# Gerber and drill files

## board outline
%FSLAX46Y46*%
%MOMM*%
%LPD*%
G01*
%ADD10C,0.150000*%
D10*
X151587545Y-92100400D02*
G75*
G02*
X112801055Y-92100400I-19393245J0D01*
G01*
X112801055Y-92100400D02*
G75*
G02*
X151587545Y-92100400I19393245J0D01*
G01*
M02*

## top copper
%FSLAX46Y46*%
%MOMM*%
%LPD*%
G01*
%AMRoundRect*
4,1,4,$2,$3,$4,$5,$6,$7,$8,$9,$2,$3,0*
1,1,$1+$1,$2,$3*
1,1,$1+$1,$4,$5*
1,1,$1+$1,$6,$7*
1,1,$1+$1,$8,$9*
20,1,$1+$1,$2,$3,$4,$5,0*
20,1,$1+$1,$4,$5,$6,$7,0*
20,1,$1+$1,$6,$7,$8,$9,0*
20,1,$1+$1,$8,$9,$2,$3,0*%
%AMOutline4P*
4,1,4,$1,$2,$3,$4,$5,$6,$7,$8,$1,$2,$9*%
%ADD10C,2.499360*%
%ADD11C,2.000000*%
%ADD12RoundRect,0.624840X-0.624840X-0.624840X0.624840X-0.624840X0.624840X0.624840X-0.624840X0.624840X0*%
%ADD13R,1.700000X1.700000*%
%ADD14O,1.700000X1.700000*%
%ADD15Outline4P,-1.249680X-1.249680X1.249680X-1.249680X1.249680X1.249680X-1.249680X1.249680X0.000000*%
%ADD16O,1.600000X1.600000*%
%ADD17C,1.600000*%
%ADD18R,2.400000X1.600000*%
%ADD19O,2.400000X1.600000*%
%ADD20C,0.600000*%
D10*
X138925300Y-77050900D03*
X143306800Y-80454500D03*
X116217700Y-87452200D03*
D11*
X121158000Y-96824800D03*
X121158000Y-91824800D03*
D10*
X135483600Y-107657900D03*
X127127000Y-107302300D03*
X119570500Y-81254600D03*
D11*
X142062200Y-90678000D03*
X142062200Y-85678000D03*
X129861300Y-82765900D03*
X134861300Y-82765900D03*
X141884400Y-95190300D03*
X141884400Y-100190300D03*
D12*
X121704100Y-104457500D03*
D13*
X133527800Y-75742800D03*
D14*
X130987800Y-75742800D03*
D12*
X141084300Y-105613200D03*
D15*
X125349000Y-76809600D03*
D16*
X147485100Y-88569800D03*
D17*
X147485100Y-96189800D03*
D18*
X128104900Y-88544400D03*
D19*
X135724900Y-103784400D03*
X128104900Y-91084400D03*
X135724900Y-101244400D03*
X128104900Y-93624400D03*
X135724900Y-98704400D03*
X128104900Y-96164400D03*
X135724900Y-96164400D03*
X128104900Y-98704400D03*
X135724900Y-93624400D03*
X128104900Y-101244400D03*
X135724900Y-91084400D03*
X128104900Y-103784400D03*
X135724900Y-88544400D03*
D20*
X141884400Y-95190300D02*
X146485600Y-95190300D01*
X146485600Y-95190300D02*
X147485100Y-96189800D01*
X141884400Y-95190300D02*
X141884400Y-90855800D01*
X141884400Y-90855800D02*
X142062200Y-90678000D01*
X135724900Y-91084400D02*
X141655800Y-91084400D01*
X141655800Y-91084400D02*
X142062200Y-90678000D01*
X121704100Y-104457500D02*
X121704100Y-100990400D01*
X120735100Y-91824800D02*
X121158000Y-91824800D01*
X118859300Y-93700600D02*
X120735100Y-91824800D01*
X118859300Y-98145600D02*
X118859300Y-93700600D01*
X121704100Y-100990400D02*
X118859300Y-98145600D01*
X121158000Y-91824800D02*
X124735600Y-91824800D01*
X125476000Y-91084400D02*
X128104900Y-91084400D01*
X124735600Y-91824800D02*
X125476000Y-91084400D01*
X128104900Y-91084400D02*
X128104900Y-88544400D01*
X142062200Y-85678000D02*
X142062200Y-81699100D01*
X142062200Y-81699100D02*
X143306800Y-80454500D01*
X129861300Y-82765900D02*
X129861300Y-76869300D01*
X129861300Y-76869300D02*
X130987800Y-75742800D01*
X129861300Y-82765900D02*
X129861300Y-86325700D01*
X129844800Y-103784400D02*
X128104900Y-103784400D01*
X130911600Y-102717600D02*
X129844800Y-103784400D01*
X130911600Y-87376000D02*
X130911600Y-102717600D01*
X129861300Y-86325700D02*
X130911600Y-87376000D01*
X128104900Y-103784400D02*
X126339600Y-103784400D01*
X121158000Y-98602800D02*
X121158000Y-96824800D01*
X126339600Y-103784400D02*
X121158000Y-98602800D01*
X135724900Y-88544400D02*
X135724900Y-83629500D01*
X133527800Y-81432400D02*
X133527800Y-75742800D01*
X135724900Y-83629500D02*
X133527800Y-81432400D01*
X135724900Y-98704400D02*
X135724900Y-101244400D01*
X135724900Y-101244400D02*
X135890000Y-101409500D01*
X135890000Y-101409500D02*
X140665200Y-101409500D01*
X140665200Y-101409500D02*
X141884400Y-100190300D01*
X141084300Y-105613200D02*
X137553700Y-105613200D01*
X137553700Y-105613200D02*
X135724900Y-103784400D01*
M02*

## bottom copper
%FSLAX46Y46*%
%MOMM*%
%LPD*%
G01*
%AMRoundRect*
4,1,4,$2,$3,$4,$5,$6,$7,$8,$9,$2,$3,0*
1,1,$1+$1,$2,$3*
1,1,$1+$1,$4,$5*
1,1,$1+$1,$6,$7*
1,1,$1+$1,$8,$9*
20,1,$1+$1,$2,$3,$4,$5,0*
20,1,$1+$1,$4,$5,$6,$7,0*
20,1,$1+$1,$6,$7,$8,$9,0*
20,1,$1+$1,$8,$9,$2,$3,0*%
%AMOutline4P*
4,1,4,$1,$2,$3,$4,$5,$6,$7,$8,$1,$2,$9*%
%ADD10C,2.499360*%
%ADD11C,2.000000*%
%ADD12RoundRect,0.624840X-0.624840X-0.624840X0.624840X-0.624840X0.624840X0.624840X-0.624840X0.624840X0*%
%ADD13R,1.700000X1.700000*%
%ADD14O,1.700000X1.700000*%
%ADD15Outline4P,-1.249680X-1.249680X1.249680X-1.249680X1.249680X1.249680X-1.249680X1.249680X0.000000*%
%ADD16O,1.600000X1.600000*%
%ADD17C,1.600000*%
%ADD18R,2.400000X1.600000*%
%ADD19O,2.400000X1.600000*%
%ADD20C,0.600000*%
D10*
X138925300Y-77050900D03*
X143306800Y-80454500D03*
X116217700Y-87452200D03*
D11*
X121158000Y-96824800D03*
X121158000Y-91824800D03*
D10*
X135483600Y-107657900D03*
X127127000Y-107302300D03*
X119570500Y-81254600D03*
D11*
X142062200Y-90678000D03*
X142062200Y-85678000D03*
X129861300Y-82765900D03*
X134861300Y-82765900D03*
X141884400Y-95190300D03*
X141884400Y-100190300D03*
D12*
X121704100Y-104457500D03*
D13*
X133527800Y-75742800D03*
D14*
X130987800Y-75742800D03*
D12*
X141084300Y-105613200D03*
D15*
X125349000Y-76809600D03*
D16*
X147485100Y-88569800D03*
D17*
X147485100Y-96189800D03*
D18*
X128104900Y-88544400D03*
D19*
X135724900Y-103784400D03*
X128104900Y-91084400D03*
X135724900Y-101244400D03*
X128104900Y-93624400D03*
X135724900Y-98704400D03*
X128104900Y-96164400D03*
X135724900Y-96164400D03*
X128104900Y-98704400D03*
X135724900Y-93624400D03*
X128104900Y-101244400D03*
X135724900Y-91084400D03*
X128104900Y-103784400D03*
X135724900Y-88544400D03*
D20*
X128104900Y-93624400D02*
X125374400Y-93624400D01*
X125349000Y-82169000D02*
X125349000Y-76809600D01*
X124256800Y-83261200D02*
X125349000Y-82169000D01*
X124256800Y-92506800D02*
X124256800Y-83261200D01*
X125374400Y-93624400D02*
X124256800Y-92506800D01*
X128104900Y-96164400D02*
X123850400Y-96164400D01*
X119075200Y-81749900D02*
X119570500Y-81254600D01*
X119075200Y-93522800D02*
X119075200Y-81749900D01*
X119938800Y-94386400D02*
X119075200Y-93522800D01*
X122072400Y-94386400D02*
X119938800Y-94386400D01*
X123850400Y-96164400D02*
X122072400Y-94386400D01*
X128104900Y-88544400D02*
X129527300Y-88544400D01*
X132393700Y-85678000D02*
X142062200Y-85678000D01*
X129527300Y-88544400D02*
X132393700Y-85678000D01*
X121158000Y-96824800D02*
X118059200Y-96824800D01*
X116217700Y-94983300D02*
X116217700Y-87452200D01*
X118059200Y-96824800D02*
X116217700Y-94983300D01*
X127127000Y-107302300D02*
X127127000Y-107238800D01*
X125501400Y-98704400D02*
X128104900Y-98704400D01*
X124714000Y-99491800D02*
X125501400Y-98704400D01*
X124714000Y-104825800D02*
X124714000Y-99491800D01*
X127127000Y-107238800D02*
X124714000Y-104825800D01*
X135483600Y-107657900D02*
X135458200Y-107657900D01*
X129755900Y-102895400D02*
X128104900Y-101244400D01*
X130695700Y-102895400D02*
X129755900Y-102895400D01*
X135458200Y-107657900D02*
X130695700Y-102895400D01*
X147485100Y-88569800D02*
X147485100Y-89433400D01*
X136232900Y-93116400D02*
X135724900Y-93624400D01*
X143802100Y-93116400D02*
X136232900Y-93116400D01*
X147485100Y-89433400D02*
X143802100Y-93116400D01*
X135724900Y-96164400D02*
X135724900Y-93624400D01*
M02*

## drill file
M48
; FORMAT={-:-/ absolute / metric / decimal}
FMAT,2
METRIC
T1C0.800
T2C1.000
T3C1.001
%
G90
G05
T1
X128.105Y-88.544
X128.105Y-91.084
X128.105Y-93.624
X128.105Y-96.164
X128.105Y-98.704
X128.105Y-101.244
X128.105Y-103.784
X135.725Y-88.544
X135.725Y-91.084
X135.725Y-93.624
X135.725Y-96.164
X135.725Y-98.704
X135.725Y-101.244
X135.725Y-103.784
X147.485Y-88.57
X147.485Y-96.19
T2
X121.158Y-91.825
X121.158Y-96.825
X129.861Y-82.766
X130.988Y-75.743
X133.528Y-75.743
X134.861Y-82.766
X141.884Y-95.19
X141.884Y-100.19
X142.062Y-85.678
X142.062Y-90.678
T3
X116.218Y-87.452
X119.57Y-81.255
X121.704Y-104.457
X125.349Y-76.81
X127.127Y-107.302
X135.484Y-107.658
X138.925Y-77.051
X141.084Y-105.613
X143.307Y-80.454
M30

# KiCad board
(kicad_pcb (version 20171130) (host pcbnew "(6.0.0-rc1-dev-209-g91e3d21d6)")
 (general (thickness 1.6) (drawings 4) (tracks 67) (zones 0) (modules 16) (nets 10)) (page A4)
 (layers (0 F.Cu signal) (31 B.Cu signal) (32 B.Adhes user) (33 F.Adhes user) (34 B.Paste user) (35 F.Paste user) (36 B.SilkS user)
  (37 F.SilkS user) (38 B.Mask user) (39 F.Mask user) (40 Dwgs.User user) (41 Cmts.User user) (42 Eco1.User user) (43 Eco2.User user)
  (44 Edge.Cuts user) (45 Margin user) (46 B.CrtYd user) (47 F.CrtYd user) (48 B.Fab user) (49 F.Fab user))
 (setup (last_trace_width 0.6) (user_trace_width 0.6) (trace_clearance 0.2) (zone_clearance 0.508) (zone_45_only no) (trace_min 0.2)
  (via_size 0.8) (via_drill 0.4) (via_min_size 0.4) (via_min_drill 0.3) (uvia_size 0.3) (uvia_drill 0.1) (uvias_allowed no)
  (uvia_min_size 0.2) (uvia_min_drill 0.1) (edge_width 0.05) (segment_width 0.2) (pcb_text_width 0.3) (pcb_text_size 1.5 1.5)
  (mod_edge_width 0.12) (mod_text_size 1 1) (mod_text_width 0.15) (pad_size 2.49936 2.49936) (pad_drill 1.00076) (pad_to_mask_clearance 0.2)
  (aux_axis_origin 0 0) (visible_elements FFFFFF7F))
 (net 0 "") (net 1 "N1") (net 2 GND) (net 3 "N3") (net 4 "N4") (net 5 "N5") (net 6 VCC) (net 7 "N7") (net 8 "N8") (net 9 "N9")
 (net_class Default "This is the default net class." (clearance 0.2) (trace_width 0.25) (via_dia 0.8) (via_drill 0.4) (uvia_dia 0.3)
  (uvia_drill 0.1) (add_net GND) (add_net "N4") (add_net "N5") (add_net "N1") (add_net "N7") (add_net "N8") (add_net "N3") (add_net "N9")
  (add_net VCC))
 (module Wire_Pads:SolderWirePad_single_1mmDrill (layer F.Cu) (at 138.9253 77.0509)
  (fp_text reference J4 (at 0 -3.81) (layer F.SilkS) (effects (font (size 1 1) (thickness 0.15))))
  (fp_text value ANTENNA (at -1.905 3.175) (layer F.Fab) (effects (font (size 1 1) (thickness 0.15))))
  (pad 1 thru_hole circle (at 0 0) (size 2.49936 2.49936) (drill 1.00076) (layers *.Cu *.Mask) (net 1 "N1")))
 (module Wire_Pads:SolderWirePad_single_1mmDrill (layer F.Cu) (at 143.3068 80.4545)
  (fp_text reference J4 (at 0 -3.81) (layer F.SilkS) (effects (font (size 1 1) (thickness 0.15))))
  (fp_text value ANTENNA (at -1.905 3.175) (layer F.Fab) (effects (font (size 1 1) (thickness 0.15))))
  (pad 1 thru_hole circle (at 0 0) (size 2.49936 2.49936) (drill 1.00076) (layers *.Cu *.Mask) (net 1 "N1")))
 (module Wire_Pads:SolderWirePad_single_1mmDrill (layer F.Cu) (at 116.2177 87.4522)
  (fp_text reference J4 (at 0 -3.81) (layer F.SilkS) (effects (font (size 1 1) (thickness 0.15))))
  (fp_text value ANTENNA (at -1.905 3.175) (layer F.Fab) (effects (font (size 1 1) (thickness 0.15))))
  (pad 1 thru_hole circle (at 0 0) (size 2.49936 2.49936) (drill 1.00076) (layers *.Cu *.Mask) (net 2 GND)))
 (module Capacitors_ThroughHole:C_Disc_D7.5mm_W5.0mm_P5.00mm (layer F.Cu) (at 121.158 96.8248 90)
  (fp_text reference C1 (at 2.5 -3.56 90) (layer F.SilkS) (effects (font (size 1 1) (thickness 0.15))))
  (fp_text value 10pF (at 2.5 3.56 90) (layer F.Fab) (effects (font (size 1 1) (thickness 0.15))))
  (pad 1 thru_hole circle (at 0 0 90) (size 2 2) (drill 1) (layers *.Cu *.Mask) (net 2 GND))
  (pad 2 thru_hole circle (at 5 0 90) (size 2 2) (drill 1) (layers *.Cu *.Mask) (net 1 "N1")))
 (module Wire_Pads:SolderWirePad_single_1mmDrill (layer F.Cu) (at 135.4836 107.6579)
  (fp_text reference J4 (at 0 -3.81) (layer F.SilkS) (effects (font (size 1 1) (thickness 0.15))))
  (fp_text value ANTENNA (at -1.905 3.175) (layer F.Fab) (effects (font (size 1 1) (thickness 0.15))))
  (pad 1 thru_hole circle (at 0 0) (size 2.49936 2.49936) (drill 1.00076) (layers *.Cu *.Mask) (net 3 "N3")))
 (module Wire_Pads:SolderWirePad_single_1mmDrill (layer F.Cu) (at 127.127 107.3023)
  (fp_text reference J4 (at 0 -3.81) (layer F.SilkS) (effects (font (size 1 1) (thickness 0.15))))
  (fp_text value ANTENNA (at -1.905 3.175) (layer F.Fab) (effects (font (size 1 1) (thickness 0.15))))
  (pad 1 thru_hole circle (at 0 0) (size 2.49936 2.49936) (drill 1.00076) (layers *.Cu *.Mask) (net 3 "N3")))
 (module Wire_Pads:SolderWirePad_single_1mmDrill (layer F.Cu) (at 119.5705 81.2546)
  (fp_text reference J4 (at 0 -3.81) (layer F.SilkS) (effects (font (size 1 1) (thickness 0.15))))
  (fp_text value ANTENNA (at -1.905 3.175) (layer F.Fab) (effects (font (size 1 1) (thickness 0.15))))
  (pad 1 thru_hole circle (at 0 0) (size 2.49936 2.49936) (drill 1.00076) (layers *.Cu *.Mask) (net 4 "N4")))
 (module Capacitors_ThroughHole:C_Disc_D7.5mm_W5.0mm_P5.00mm (layer F.Cu) (at 142.0622 90.678 90)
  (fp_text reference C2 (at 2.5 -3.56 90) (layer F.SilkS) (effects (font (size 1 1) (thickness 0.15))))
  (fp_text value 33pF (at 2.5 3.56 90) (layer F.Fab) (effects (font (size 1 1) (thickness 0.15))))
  (pad 1 thru_hole circle (at 0 0 90) (size 2 2) (drill 1) (layers *.Cu *.Mask) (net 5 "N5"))
  (pad 2 thru_hole circle (at 5 0 90) (size 2 2) (drill 1) (layers *.Cu *.Mask) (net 1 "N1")))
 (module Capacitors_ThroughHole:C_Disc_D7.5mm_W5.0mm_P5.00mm (layer F.Cu) (at 134.8613 82.7659 180)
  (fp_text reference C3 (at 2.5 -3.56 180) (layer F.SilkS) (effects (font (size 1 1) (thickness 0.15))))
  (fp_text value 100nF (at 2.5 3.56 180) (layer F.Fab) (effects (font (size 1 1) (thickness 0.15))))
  (pad 2 thru_hole circle (at 5 0 180) (size 2 2) (drill 1) (layers *.Cu *.Mask) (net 2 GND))
  (pad 1 thru_hole circle (at 0 0 180) (size 2 2) (drill 1) (layers *.Cu *.Mask) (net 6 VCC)))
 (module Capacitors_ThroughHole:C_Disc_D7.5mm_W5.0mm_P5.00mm (layer F.Cu) (at 141.8844 100.1903 90)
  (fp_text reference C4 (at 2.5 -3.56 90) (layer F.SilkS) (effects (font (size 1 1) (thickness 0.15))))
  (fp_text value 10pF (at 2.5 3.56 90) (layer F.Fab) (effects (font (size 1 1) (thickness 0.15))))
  (pad 2 thru_hole circle (at 5 0 90) (size 2 2) (drill 1) (layers *.Cu *.Mask) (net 5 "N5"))
  (pad 1 thru_hole circle (at 0 0 90) (size 2 2) (drill 1) (layers *.Cu *.Mask) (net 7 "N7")))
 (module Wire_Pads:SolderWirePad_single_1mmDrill (layer F.Cu) (at 121.7041 104.4575)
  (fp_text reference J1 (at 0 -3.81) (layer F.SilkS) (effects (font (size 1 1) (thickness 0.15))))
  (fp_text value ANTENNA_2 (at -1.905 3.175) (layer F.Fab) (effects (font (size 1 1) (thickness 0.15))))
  (pad 1 thru_hole roundrect (at 0 0) (size 2.49936 2.49936) (drill 1.00076) (layers *.Cu *.Mask) (roundrect_rratio 0.25) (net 1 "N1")))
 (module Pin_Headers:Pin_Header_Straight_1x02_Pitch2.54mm (layer F.Cu) (at 133.5278 75.7428 270)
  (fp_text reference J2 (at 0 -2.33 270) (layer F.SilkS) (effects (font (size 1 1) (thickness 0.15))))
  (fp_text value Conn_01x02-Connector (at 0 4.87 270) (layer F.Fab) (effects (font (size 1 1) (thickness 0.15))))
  (pad 1 thru_hole rect (at 0 0 270) (size 1.7 1.7) (drill 1) (layers *.Cu *.Mask) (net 6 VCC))
  (pad 2 thru_hole oval (at 0 2.54 270) (size 1.7 1.7) (drill 1) (layers *.Cu *.Mask) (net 2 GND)))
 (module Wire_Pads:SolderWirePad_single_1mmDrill (layer F.Cu) (at 141.0843 105.6132)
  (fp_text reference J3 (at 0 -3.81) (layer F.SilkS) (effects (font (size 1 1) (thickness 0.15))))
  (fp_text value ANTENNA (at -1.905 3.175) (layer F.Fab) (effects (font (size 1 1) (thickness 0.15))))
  (pad 1 thru_hole roundrect (at 0 0) (size 2.49936 2.49936) (drill 1.00076) (layers *.Cu *.Mask) (roundrect_rratio 0.25) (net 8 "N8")))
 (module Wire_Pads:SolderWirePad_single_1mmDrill (layer F.Cu) (at 125.349 76.8096)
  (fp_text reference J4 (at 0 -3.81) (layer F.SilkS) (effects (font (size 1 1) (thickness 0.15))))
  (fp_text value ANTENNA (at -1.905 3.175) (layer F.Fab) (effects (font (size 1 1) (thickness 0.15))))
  (pad 1 thru_hole trapezoid (at 0 0) (size 2.49936 2.49936) (drill 1.00076) (layers *.Cu *.Mask) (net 4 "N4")))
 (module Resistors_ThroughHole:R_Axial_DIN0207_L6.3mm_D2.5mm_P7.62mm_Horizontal (layer F.Cu) (at 147.4851 96.1898 90)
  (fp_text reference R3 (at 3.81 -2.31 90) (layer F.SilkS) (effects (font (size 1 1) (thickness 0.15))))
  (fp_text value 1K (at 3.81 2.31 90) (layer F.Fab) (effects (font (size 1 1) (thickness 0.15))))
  (pad 2 thru_hole oval (at 7.62 0 90) (size 1.6 1.6) (drill 0.8) (layers *.Cu *.Mask) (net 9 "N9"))
  (pad 1 thru_hole circle (at 0 0 90) (size 1.6 1.6) (drill 0.8) (layers *.Cu *.Mask) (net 5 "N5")))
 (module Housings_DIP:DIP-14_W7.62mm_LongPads (layer F.Cu) (at 128.1049 88.5444)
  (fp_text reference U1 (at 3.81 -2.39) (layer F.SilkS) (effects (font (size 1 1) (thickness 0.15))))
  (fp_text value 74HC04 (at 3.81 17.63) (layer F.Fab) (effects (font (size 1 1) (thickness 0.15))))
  (pad 1 thru_hole rect (at 0 0) (size 2.4 1.6) (drill 0.8) (layers *.Cu *.Mask) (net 1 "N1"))
  (pad 8 thru_hole oval (at 7.62 15.24) (size 2.4 1.6) (drill 0.8) (layers *.Cu *.Mask) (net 8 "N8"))
  (pad 2 thru_hole oval (at 0 2.54) (size 2.4 1.6) (drill 0.8) (layers *.Cu *.Mask) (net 1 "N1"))
  (pad 9 thru_hole oval (at 7.62 12.7) (size 2.4 1.6) (drill 0.8) (layers *.Cu *.Mask) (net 7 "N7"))
  (pad 3 thru_hole oval (at 0 5.08) (size 2.4 1.6) (drill 0.8) (layers *.Cu *.Mask) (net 4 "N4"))
  (pad 10 thru_hole oval (at 7.62 10.16) (size 2.4 1.6) (drill 0.8) (layers *.Cu *.Mask) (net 7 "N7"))
  (pad 4 thru_hole oval (at 0 7.62) (size 2.4 1.6) (drill 0.8) (layers *.Cu *.Mask) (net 4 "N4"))
  (pad 11 thru_hole oval (at 7.62 7.62) (size 2.4 1.6) (drill 0.8) (layers *.Cu *.Mask) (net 9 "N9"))
  (pad 5 thru_hole oval (at 0 10.16) (size 2.4 1.6) (drill 0.8) (layers *.Cu *.Mask) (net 3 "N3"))
  (pad 12 thru_hole oval (at 7.62 5.08) (size 2.4 1.6) (drill 0.8) (layers *.Cu *.Mask) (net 9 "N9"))
  (pad 6 thru_hole oval (at 0 12.7) (size 2.4 1.6) (drill 0.8) (layers *.Cu *.Mask) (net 3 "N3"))
  (pad 13 thru_hole oval (at 7.62 2.54) (size 2.4 1.6) (drill 0.8) (layers *.Cu *.Mask) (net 5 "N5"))
  (pad 7 thru_hole oval (at 0 15.24) (size 2.4 1.6) (drill 0.8) (layers *.Cu *.Mask) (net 2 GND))
  (pad 14 thru_hole oval (at 7.62 0) (size 2.4 1.6) (drill 0.8) (layers *.Cu *.Mask) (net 6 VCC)))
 (gr_circle (center 132.1943 92.1004) (end 151.587545 92.1004) (layer Edge.Cuts) (width 0.15))
 (segment (start 128.1049 93.6244) (end 125.3744 93.6244) (width 0.6) (layer B.Cu) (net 4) (status 400000))
 (segment (start 125.349 82.169) (end 125.349 76.8096) (width 0.6) (layer B.Cu) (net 4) (status 800000))
 (segment (start 124.2568 83.2612) (end 125.349 82.169) (width 0.6) (layer B.Cu) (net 4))
 (segment (start 124.2568 92.5068) (end 124.2568 83.2612) (width 0.6) (layer B.Cu) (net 4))
 (segment (start 125.3744 93.6244) (end 124.2568 92.5068) (width 0.6) (layer B.Cu) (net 4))
 (segment (start 128.1049 96.1644) (end 123.8504 96.1644) (width 0.6) (layer B.Cu) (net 4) (status 400000))
 (segment (start 119.0752 81.7499) (end 119.5705 81.2546) (width 0.6) (layer B.Cu) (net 4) (status C00000))
 (segment (start 119.0752 93.5228) (end 119.0752 81.7499) (width 0.6) (layer B.Cu) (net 4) (status 800000))
 (segment (start 119.9388 94.3864) (end 119.0752 93.5228) (width 0.6) (layer B.Cu) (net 4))
 (segment (start 122.0724 94.3864) (end 119.9388 94.3864) (width 0.6) (layer B.Cu) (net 4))
 (segment (start 123.8504 96.1644) (end 122.0724 94.3864) (width 0.6) (layer B.Cu) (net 4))
 (segment (start 141.8844 95.1903) (end 146.4856 95.1903) (width 0.6) (layer F.Cu) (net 5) (status 400000))
 (segment (start 146.4856 95.1903) (end 147.4851 96.1898) (width 0.6) (layer F.Cu) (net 5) (status 800000))
 (segment (start 141.8844 95.1903) (end 141.8844 90.8558) (width 0.6) (layer F.Cu) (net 5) (status C00000))
 (segment (start 141.8844 90.8558) (end 142.0622 90.678) (width 0.6) (layer F.Cu) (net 5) (status C00000))
 (segment (start 135.7249 91.0844) (end 141.6558 91.0844) (width 0.6) (layer F.Cu) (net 5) (status C00000))
 (segment (start 141.6558 91.0844) (end 142.0622 90.678) (width 0.6) (layer F.Cu) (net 5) (status C00000))
 (segment (start 121.7041 104.4575) (end 121.7041 100.9904) (width 0.6) (layer F.Cu) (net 1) (status 400000))
 (segment (start 120.7351 91.8248) (end 121.158 91.8248) (width 0.6) (layer F.Cu) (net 1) (status C00000))
 (segment (start 118.8593 93.7006) (end 120.7351 91.8248) (width 0.6) (layer F.Cu) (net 1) (status 800000))
 (segment (start 118.8593 98.1456) (end 118.8593 93.7006) (width 0.6) (layer F.Cu) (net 1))
 (segment (start 121.7041 100.9904) (end 118.8593 98.1456) (width 0.6) (layer F.Cu) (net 1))
 (segment (start 121.158 91.8248) (end 124.7356 91.8248) (width 0.6) (layer F.Cu) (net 1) (status 400000))
 (segment (start 125.476 91.0844) (end 128.1049 91.0844) (width 0.6) (layer F.Cu) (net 1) (status 800000))
 (segment (start 124.7356 91.8248) (end 125.476 91.0844) (width 0.6) (layer F.Cu) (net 1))
 (segment (start 128.1049 91.0844) (end 128.1049 88.5444) (width 0.6) (layer F.Cu) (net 1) (status C00000))
 (segment (start 128.1049 88.5444) (end 129.5273 88.5444) (width 0.6) (layer B.Cu) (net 1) (status 400000))
 (segment (start 132.3937 85.678) (end 142.0622 85.678) (width 0.6) (layer B.Cu) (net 1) (status 800000))
 (segment (start 129.5273 88.5444) (end 132.3937 85.678) (width 0.6) (layer B.Cu) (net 1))
 (segment (start 142.0622 85.678) (end 142.0622 81.6991) (width 0.6) (layer F.Cu) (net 1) (status 400000))
 (segment (start 142.0622 81.6991) (end 143.3068 80.4545) (width 0.6) (layer F.Cu) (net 1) (status 800000))
 (segment (start 129.8613 82.7659) (end 129.8613 76.8693) (width 0.6) (layer F.Cu) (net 2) (status 400000))
 (segment (start 129.8613 76.8693) (end 130.9878 75.7428) (width 0.6) (layer F.Cu) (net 2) (status 800000))
 (segment (start 129.8613 82.7659) (end 129.8613 86.3257) (width 0.6) (layer F.Cu) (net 2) (status 400000))
 (segment (start 129.8448 103.7844) (end 128.1049 103.7844) (width 0.6) (layer F.Cu) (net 2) (status 800000))
 (segment (start 130.9116 102.7176) (end 129.8448 103.7844) (width 0.6) (layer F.Cu) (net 2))
 (segment (start 130.9116 87.376) (end 130.9116 102.7176) (width 0.6) (layer F.Cu) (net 2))
 (segment (start 129.8613 86.3257) (end 130.9116 87.376) (width 0.6) (layer F.Cu) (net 2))
 (segment (start 128.1049 103.7844) (end 126.3396 103.7844) (width 0.6) (layer F.Cu) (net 2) (status 400000))
 (segment (start 121.158 98.6028) (end 121.158 96.8248) (width 0.6) (layer F.Cu) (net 2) (status 800000))
 (segment (start 126.3396 103.7844) (end 121.158 98.6028) (width 0.6) (layer F.Cu) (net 2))
 (segment (start 121.158 96.8248) (end 118.0592 96.8248) (width 0.6) (layer B.Cu) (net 2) (status 400000))
 (segment (start 116.2177 94.9833) (end 116.2177 87.4522) (width 0.6) (layer B.Cu) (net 2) (status 800000))
 (segment (start 118.0592 96.8248) (end 116.2177 94.9833) (width 0.6) (layer B.Cu) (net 2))
 (segment (start 135.7249 88.5444) (end 135.7249 83.6295) (width 0.6) (layer F.Cu) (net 6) (status 400000))
 (segment (start 133.5278 81.4324) (end 133.5278 75.7428) (width 0.6) (layer F.Cu) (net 6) (status 800000))
 (segment (start 135.7249 83.6295) (end 133.5278 81.4324) (width 0.6) (layer F.Cu) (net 6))
 (segment (start 135.7249 98.7044) (end 135.7249 101.2444) (width 0.6) (layer F.Cu) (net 7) (status C00000))
 (segment (start 135.7249 101.2444) (end 135.89 101.4095) (width 0.6) (layer F.Cu) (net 7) (status C00000))
 (segment (start 135.89 101.4095) (end 140.6652 101.4095) (width 0.6) (layer F.Cu) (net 7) (status 400000))
 (segment (start 140.6652 101.4095) (end 141.8844 100.1903) (width 0.6) (layer F.Cu) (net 7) (status 800000))
 (segment (start 141.0843 105.6132) (end 137.5537 105.6132) (width 0.6) (layer F.Cu) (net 8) (status 400000))
 (segment (start 137.5537 105.6132) (end 135.7249 103.7844) (width 0.6) (layer F.Cu) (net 8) (status 800000))
 (segment (start 127.127 107.3023) (end 127.127 107.2388) (width 0.6) (layer B.Cu) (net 3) (status C00000))
 (segment (start 125.5014 98.7044) (end 128.1049 98.7044) (width 0.6) (layer B.Cu) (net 3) (status 800000))
 (segment (start 124.714 99.4918) (end 125.5014 98.7044) (width 0.6) (layer B.Cu) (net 3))
 (segment (start 124.714 104.8258) (end 124.714 99.4918) (width 0.6) (layer B.Cu) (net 3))
 (segment (start 127.127 107.2388) (end 124.714 104.8258) (width 0.6) (layer B.Cu) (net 3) (status 400000))
 (segment (start 135.4836 107.6579) (end 135.4582 107.6579) (width 0.6) (layer B.Cu) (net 3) (status C00000))
 (segment (start 129.7559 102.8954) (end 128.1049 101.2444) (width 0.6) (layer B.Cu) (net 3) (status 800000))
 (segment (start 130.6957 102.8954) (end 129.7559 102.8954) (width 0.6) (layer B.Cu) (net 3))
 (segment (start 135.4582 107.6579) (end 130.6957 102.8954) (width 0.6) (layer B.Cu) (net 3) (status 400000))
 (segment (start 147.4851 88.5698) (end 147.4851 89.4334) (width 0.6) (layer B.Cu) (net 9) (status 400000))
 (segment (start 136.2329 93.1164) (end 135.7249 93.6244) (width 0.6) (layer B.Cu) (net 9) (status C00000))
 (segment (start 143.8021 93.1164) (end 136.2329 93.1164) (width 0.6) (layer B.Cu) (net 9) (status 800000))
 (segment (start 147.4851 89.4334) (end 143.8021 93.1164) (width 0.6) (layer B.Cu) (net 9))
 (segment (start 135.7249 96.1644) (end 135.7249 93.6244) (width 0.6) (layer B.Cu) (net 9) (status C00000)))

